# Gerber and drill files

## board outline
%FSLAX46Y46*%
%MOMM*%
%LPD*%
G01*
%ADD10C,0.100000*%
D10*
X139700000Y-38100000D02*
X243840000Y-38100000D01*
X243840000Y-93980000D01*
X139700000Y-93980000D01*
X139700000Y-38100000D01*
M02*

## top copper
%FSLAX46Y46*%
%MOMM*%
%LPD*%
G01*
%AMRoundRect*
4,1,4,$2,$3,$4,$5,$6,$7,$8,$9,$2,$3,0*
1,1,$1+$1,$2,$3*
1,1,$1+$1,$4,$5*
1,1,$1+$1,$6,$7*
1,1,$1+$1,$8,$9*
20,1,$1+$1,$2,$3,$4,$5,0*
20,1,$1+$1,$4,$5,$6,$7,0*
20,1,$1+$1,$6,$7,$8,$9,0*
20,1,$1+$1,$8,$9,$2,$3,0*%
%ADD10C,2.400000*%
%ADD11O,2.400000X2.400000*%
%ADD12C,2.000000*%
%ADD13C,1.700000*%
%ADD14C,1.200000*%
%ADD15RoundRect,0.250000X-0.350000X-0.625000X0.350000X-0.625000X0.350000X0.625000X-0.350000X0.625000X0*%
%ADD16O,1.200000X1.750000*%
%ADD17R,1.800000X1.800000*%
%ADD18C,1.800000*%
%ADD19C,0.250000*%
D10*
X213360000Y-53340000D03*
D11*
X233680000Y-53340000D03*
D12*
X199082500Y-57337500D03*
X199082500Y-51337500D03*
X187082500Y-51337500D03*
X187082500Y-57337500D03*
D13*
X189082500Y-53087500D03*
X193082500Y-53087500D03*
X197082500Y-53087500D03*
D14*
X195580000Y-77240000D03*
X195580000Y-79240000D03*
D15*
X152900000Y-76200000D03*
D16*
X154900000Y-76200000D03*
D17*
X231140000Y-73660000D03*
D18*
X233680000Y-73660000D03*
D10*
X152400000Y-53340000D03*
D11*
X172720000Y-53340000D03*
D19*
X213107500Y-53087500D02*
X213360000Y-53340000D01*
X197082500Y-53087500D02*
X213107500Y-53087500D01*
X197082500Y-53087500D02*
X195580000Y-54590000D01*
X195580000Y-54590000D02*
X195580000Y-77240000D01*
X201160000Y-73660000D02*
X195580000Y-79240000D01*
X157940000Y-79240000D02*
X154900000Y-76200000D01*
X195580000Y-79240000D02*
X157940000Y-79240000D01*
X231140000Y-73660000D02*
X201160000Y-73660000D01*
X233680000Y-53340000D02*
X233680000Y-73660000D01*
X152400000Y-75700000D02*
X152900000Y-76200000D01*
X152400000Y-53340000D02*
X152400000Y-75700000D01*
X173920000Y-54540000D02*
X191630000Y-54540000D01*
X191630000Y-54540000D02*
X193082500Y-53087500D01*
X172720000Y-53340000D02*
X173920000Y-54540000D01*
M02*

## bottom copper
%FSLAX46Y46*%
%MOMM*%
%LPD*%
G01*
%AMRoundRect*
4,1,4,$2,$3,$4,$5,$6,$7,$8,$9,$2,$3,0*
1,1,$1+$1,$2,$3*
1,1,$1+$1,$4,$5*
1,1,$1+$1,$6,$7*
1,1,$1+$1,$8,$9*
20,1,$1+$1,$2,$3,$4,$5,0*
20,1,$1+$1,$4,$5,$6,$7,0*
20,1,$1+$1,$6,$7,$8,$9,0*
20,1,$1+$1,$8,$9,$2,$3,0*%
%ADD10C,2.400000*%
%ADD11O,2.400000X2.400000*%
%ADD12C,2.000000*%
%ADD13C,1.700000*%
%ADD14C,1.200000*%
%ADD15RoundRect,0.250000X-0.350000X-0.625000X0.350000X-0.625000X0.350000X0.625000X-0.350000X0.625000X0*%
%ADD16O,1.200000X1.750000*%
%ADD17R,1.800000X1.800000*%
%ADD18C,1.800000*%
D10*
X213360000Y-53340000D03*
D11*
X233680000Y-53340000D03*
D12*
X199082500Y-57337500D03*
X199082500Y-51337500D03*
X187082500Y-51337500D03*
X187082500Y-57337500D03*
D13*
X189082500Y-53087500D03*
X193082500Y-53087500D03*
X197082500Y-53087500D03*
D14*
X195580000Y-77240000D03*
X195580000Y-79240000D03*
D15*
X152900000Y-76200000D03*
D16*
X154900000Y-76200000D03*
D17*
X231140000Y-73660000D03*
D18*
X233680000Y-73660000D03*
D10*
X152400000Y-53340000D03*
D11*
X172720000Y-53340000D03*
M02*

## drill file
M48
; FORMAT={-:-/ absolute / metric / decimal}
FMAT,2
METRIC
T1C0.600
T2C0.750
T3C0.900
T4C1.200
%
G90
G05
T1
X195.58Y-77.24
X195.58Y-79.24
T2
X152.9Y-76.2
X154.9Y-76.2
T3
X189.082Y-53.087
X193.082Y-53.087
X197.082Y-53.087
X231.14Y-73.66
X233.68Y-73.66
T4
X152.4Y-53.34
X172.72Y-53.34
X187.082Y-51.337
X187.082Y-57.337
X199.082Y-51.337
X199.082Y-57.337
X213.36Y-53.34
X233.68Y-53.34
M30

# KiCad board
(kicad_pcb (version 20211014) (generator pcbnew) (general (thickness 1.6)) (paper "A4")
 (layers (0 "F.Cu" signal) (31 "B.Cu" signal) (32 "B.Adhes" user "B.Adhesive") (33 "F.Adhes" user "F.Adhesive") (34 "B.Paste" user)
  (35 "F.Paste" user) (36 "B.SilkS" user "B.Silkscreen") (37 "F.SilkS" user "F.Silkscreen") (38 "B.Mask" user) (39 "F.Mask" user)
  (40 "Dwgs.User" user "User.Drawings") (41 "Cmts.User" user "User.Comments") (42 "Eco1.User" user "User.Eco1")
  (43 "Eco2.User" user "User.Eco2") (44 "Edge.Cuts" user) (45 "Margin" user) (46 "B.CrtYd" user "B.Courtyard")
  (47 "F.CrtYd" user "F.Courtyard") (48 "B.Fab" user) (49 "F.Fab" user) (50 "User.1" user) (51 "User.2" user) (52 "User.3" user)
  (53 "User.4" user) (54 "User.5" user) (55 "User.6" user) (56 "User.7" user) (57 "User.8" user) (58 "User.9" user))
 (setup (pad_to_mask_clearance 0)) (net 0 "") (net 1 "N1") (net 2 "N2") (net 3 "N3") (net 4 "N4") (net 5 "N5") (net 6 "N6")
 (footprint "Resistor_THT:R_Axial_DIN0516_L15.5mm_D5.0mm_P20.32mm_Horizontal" (layer "F.Cu") (at 213.36 53.34)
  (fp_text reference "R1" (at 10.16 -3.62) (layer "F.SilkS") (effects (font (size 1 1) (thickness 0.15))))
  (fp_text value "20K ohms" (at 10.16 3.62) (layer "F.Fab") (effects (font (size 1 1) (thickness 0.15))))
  (pad "1" thru_hole circle (at 0 0) (size 2.4 2.4) (drill 1.2) (layers *.Cu *.Mask) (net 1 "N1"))
  (pad "2" thru_hole oval (at 20.32 0) (size 2.4 2.4) (drill 1.2) (layers *.Cu *.Mask) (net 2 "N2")))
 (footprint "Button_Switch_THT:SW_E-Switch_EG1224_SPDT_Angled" (layer "F.Cu") (at 189.0825 53.0875)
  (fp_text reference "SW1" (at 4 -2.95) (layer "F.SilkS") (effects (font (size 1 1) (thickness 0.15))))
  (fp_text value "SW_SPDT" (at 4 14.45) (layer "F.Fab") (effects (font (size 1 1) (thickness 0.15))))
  (pad "" thru_hole circle (at 10 4.25) (size 2 2) (drill 1.2) (layers *.Cu *.Mask))
  (pad "" thru_hole circle (at 10 -1.75) (size 2 2) (drill 1.2) (layers *.Cu *.Mask))
  (pad "" thru_hole circle (at -2 -1.75) (size 2 2) (drill 1.2) (layers *.Cu *.Mask))
  (pad "" thru_hole circle (at -2 4.25) (size 2 2) (drill 1.2) (layers *.Cu *.Mask))
  (pad "1" thru_hole circle (at 0 0) (size 1.7 1.7) (drill 0.9) (layers *.Cu *.Mask) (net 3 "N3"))
  (pad "2" thru_hole circle (at 4 0) (size 1.7 1.7) (drill 0.9) (layers *.Cu *.Mask) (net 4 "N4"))
  (pad "3" thru_hole circle (at 8 0) (size 1.7 1.7) (drill 0.9) (layers *.Cu *.Mask) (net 1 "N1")))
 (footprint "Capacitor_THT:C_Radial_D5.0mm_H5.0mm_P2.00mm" (layer "F.Cu") (at 195.58 77.24 -90)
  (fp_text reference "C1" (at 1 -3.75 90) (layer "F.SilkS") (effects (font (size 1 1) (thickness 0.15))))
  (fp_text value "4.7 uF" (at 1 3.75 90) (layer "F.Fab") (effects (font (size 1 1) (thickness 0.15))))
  (pad "1" thru_hole circle (at 0 0 270) (size 1.2 1.2) (drill 0.6) (layers *.Cu *.Mask) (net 1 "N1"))
  (pad "2" thru_hole circle (at 2 0 270) (size 1.2 1.2) (drill 0.6) (layers *.Cu *.Mask) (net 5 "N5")))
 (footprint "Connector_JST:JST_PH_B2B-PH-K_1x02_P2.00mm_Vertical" (layer "F.Cu") (at 152.9 76.2)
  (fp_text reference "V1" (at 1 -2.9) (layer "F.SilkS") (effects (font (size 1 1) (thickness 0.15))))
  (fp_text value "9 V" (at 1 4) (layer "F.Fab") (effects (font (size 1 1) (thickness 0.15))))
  (pad "1" thru_hole roundrect (at 0 0) (size 1.2 1.75) (drill 0.75) (layers *.Cu *.Mask) (roundrect_rratio 0.208333) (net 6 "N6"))
  (pad "2" thru_hole oval (at 2 0) (size 1.2 1.75) (drill 0.75) (layers *.Cu *.Mask) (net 5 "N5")))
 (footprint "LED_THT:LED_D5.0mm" (layer "F.Cu") (at 231.14 73.66)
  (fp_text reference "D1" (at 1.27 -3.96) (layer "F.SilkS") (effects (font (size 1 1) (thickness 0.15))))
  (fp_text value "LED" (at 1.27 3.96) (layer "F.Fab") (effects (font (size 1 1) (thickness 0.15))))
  (pad "1" thru_hole rect (at 0 0) (size 1.8 1.8) (drill 0.9) (layers *.Cu *.Mask) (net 5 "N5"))
  (pad "2" thru_hole circle (at 2.54 0) (size 1.8 1.8) (drill 0.9) (layers *.Cu *.Mask) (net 2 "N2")))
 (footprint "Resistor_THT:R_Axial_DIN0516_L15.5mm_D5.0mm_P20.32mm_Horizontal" (layer "F.Cu") (at 152.4 53.34)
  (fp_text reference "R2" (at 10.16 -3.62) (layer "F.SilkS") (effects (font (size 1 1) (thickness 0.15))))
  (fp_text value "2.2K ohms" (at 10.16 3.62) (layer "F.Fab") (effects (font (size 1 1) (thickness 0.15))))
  (pad "1" thru_hole circle (at 0 0) (size 2.4 2.4) (drill 1.2) (layers *.Cu *.Mask) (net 6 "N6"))
  (pad "2" thru_hole oval (at 20.32 0) (size 2.4 2.4) (drill 1.2) (layers *.Cu *.Mask) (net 4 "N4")))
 (gr_rect (start 139.7 38.1) (end 243.84 93.98) (layer "Edge.Cuts") (width 0.1) (fill none))
 (segment (start 213.1075 53.0875) (end 213.36 53.34) (width 0.25) (layer "F.Cu") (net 1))
 (segment (start 197.0825 53.0875) (end 213.1075 53.0875) (width 0.25) (layer "F.Cu") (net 1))
 (segment (start 197.0825 53.0875) (end 195.58 54.59) (width 0.25) (layer "F.Cu") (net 1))
 (segment (start 195.58 54.59) (end 195.58 77.24) (width 0.25) (layer "F.Cu") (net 1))
 (segment (start 201.16 73.66) (end 195.58 79.24) (width 0.25) (layer "F.Cu") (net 5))
 (segment (start 157.94 79.24) (end 154.9 76.2) (width 0.25) (layer "F.Cu") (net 5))
 (segment (start 195.58 79.24) (end 157.94 79.24) (width 0.25) (layer "F.Cu") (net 5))
 (segment (start 231.14 73.66) (end 201.16 73.66) (width 0.25) (layer "F.Cu") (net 5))
 (segment (start 233.68 53.34) (end 233.68 73.66) (width 0.25) (layer "F.Cu") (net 2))
 (segment (start 152.4 75.7) (end 152.9 76.2) (width 0.25) (layer "F.Cu") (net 6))
 (segment (start 152.4 53.34) (end 152.4 75.7) (width 0.25) (layer "F.Cu") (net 6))
 (segment (start 173.92 54.54) (end 191.63 54.54) (width 0.25) (layer "F.Cu") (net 4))
 (segment (start 191.63 54.54) (end 193.0825 53.0875) (width 0.25) (layer "F.Cu") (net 4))
 (segment (start 172.72 53.34) (end 173.92 54.54) (width 0.25) (layer "F.Cu") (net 4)))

